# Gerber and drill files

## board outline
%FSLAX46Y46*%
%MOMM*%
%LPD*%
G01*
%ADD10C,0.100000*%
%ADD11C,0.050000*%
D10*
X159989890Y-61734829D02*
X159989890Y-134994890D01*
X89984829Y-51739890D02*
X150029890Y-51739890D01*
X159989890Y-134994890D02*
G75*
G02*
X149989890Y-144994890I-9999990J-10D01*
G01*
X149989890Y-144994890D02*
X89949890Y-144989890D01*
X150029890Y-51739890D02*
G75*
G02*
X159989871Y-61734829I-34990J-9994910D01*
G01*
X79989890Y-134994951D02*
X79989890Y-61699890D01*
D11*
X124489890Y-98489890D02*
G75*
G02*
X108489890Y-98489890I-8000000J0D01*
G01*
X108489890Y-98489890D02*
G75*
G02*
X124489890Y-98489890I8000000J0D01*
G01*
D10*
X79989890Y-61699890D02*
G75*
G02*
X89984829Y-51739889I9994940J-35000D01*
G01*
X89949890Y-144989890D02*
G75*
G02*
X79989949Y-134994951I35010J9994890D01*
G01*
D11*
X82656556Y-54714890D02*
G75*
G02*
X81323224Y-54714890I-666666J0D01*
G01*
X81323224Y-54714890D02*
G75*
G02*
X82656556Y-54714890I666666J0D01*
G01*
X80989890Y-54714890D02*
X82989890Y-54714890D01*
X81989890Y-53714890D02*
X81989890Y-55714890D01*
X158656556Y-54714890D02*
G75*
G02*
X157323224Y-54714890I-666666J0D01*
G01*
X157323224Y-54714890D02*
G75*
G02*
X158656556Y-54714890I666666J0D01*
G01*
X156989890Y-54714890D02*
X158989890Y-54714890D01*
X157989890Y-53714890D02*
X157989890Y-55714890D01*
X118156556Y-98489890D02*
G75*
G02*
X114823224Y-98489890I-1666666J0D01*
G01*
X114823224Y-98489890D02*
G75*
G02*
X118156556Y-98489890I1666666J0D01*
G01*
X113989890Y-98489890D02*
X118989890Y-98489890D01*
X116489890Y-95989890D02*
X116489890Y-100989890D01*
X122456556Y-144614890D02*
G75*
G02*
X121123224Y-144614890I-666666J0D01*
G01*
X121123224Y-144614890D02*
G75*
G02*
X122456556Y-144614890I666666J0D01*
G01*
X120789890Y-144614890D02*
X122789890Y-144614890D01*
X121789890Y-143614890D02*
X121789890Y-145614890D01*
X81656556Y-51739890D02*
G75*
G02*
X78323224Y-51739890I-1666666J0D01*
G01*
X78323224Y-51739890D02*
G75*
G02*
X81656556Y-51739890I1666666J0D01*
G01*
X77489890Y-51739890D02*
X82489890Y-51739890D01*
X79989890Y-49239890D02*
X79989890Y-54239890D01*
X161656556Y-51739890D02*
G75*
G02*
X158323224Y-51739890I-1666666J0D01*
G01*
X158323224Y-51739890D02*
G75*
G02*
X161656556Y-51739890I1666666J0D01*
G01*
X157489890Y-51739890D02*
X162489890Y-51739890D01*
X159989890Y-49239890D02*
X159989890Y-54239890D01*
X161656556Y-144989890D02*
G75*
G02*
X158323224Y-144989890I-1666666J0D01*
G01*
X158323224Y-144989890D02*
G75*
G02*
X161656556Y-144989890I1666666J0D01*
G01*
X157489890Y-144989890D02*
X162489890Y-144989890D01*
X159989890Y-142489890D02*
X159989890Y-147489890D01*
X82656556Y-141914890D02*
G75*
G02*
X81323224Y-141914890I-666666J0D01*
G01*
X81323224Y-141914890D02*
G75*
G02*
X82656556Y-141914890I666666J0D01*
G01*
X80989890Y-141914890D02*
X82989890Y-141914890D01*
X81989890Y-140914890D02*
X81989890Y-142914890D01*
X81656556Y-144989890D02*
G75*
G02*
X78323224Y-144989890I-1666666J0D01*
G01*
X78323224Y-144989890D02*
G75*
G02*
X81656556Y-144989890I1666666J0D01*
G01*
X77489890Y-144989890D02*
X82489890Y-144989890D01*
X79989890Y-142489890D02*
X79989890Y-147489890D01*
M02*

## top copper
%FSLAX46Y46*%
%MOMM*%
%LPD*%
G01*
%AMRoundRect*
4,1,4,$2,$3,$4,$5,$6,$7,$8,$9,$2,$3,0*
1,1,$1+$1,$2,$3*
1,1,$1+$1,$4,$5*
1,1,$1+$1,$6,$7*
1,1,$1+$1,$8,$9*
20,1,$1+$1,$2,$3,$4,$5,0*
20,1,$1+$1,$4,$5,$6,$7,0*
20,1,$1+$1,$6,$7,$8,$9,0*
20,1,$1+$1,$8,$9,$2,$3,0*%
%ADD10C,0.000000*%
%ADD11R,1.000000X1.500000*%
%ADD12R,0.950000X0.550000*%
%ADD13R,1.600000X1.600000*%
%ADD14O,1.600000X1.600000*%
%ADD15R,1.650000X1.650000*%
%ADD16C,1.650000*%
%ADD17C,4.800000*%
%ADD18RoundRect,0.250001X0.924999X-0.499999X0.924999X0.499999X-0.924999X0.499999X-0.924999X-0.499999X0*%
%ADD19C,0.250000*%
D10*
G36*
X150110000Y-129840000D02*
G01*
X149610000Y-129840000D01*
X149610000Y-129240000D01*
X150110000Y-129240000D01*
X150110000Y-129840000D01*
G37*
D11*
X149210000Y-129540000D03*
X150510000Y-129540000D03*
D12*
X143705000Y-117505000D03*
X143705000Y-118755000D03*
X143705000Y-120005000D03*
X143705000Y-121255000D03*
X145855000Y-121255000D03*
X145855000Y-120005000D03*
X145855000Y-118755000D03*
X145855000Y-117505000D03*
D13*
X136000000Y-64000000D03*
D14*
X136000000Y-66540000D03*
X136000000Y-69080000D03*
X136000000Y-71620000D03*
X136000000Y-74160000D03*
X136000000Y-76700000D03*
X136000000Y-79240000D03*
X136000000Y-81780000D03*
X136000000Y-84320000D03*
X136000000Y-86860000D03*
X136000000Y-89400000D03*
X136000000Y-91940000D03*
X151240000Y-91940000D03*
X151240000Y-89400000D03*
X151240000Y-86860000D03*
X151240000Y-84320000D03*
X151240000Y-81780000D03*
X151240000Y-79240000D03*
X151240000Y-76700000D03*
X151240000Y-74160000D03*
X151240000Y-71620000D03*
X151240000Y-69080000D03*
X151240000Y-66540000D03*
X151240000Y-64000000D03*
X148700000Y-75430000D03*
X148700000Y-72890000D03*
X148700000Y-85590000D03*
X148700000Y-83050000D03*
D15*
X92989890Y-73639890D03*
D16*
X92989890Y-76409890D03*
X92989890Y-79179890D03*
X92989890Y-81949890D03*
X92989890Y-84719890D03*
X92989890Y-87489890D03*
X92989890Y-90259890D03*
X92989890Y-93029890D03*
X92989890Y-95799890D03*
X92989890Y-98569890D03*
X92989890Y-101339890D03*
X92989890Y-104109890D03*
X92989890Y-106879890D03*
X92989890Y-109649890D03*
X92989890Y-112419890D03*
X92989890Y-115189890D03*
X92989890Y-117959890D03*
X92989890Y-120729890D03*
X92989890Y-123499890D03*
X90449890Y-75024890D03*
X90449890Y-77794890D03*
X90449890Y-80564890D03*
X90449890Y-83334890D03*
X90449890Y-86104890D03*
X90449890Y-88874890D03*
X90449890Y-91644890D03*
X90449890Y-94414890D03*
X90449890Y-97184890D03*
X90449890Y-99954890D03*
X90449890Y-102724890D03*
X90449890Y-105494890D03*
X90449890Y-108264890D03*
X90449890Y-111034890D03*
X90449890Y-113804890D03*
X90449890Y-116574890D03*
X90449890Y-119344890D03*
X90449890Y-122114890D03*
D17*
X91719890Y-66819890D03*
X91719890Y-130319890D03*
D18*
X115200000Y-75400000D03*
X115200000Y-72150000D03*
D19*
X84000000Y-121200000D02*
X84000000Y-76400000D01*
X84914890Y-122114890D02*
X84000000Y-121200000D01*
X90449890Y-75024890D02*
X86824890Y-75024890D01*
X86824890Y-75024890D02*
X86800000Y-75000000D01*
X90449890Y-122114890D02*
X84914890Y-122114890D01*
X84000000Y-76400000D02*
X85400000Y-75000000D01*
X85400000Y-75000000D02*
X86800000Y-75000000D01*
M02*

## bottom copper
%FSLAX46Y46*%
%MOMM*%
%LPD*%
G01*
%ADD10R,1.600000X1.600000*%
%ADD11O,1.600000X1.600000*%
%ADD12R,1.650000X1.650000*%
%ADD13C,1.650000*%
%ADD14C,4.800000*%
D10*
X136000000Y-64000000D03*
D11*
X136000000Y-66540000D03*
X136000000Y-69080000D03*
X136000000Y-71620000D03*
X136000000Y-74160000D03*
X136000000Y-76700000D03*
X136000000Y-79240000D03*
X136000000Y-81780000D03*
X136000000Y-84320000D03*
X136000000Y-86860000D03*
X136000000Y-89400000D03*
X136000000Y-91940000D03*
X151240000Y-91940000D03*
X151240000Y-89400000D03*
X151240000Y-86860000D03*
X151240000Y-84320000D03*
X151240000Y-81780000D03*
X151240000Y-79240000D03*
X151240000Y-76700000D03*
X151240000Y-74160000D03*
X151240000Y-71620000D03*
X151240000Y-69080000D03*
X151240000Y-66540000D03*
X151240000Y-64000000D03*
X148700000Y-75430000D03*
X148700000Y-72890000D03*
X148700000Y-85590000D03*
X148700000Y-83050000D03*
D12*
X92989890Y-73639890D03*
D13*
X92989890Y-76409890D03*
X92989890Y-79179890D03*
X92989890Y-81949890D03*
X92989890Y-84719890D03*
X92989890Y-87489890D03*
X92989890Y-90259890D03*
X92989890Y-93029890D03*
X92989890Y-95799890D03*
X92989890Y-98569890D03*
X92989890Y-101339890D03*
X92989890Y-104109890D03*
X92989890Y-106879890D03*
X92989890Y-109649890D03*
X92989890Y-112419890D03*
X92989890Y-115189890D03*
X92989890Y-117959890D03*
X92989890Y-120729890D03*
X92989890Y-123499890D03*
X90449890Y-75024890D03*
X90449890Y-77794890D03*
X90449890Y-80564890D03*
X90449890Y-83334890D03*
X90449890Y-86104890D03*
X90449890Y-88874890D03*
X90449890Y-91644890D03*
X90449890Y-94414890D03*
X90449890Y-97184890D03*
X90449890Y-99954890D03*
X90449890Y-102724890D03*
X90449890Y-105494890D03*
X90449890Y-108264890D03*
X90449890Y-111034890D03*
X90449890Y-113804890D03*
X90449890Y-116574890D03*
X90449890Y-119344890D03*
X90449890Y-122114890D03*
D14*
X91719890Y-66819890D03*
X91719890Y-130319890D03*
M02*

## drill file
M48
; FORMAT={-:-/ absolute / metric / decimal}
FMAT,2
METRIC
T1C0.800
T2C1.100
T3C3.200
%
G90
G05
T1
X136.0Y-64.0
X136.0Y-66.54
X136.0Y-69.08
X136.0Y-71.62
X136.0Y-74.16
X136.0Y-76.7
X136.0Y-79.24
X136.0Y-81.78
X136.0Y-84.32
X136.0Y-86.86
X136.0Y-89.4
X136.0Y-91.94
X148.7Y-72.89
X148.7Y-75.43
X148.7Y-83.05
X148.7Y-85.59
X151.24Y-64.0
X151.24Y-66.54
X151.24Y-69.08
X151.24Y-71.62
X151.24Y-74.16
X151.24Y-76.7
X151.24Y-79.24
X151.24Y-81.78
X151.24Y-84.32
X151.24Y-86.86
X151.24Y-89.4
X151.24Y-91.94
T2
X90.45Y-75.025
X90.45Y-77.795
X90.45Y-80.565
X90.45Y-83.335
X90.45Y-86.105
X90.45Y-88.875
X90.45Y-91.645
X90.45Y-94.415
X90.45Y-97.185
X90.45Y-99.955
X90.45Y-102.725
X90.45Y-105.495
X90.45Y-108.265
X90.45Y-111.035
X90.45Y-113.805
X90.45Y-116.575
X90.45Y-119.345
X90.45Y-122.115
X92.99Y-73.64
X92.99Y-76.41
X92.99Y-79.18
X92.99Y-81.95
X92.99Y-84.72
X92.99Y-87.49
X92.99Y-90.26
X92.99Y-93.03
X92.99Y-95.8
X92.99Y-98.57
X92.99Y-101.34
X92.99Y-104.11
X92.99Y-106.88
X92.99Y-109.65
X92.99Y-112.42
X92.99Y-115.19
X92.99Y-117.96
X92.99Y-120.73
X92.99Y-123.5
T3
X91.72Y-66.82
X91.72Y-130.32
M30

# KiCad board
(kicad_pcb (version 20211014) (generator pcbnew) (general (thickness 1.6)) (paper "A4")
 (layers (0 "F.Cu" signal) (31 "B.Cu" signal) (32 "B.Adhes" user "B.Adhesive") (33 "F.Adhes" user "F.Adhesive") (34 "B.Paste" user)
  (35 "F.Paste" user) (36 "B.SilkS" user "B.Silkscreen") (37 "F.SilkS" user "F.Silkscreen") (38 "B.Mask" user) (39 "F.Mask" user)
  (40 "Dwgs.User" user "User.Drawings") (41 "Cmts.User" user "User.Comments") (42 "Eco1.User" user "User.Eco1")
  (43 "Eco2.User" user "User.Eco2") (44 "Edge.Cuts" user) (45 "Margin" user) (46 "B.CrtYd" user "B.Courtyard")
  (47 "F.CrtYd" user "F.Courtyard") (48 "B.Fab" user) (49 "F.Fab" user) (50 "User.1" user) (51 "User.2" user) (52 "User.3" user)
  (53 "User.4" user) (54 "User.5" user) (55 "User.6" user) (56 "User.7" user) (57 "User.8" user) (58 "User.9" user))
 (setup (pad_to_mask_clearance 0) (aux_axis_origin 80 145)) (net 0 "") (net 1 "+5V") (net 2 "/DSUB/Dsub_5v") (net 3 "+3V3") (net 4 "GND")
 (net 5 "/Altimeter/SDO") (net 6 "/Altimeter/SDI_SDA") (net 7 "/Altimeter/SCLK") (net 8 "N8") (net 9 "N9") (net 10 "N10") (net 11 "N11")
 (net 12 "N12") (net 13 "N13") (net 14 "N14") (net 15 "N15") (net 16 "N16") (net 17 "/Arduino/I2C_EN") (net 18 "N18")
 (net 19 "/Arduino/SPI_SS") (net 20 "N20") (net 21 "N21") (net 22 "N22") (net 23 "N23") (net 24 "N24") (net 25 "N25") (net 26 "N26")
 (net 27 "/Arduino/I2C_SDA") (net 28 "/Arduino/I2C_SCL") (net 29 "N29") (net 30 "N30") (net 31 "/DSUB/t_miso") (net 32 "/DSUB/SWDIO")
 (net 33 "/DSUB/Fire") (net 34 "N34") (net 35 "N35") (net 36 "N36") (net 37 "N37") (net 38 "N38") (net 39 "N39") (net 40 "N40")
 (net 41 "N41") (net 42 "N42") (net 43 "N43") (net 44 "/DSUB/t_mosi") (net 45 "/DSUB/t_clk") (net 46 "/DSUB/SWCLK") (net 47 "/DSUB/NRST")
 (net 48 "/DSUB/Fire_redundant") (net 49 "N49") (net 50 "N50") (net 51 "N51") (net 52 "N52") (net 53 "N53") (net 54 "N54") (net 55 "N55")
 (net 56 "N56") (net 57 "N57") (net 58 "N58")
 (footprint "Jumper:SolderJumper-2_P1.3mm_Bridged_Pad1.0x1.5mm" (layer "F.Cu") (at 149.86 129.54)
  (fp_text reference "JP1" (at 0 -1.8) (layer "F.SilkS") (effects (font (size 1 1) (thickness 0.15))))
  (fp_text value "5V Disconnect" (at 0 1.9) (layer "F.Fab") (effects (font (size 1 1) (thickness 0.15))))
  (fp_poly (pts (xy -0.25 -0.3) (xy 0.25 -0.3) (xy 0.25 0.3) (xy -0.25 0.3)) (layer "F.Cu") (width 0) (fill solid))
  (pad "1" smd rect (at -0.65 0) (size 1 1.5) (layers "F.Cu" "F.Mask") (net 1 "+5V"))
  (pad "2" smd rect (at 0.65 0) (size 1 1.5) (layers "F.Cu" "F.Mask") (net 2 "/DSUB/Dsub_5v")))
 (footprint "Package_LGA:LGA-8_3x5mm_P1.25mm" (layer "F.Cu") (at 144.78 119.38)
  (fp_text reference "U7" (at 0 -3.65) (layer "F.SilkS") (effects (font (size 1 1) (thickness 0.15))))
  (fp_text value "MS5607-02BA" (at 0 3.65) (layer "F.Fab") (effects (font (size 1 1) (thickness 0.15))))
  (pad "1" smd rect (at -1.075 -1.875) (size 0.95 0.55) (layers "F.Cu" "F.Paste" "F.Mask") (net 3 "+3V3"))
  (pad "2" smd rect (at -1.075 -0.625) (size 0.95 0.55) (layers "F.Cu" "F.Paste" "F.Mask") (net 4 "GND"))
  (pad "3" smd rect (at -1.075 0.625) (size 0.95 0.55) (layers "F.Cu" "F.Paste" "F.Mask") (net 4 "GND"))
  (pad "4" smd rect (at -1.075 1.875) (size 0.95 0.55) (layers "F.Cu" "F.Paste" "F.Mask") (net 4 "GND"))
  (pad "5" smd rect (at 1.075 1.875) (size 0.95 0.55) (layers "F.Cu" "F.Paste" "F.Mask") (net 4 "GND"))
  (pad "6" smd rect (at 1.075 0.625) (size 0.95 0.55) (layers "F.Cu" "F.Paste" "F.Mask") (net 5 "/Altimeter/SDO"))
  (pad "7" smd rect (at 1.075 -0.625) (size 0.95 0.55) (layers "F.Cu" "F.Paste" "F.Mask") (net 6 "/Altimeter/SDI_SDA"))
  (pad "8" smd rect (at 1.075 -1.875) (size 0.95 0.55) (layers "F.Cu" "F.Paste" "F.Mask") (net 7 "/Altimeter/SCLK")))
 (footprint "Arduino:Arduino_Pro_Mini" (layer "F.Cu") (at 136 64)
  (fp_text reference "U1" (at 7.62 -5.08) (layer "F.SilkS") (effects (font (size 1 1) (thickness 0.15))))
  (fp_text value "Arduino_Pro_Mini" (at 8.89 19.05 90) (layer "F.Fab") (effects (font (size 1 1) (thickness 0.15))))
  (pad "1" thru_hole rect locked (at 0 0) (size 1.6 1.6) (drill 0.8) (layers *.Cu *.Mask) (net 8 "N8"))
  (pad "2" thru_hole oval locked (at 0 2.54) (size 1.6 1.6) (drill 0.8) (layers *.Cu *.Mask) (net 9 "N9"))
  (pad "3" thru_hole oval locked (at 0 5.08) (size 1.6 1.6) (drill 0.8) (layers *.Cu *.Mask) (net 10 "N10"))
  (pad "4" thru_hole oval locked (at 0 7.62) (size 1.6 1.6) (drill 0.8) (layers *.Cu *.Mask) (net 4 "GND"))
  (pad "5" thru_hole oval locked (at 0 10.16) (size 1.6 1.6) (drill 0.8) (layers *.Cu *.Mask) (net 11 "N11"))
  (pad "6" thru_hole oval locked (at 0 12.7) (size 1.6 1.6) (drill 0.8) (layers *.Cu *.Mask) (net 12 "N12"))
  (pad "7" thru_hole oval locked (at 0 15.24) (size 1.6 1.6) (drill 0.8) (layers *.Cu *.Mask) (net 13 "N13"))
  (pad "8" thru_hole oval locked (at 0 17.78) (size 1.6 1.6) (drill 0.8) (layers *.Cu *.Mask) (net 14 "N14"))
  (pad "9" thru_hole oval locked (at 0 20.32) (size 1.6 1.6) (drill 0.8) (layers *.Cu *.Mask) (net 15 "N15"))
  (pad "10" thru_hole oval locked (at 0 22.86) (size 1.6 1.6) (drill 0.8) (layers *.Cu *.Mask) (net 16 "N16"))
  (pad "11" thru_hole oval locked (at 0 25.4) (size 1.6 1.6) (drill 0.8) (layers *.Cu *.Mask) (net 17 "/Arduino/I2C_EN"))
  (pad "12" thru_hole oval locked (at 0 27.94) (size 1.6 1.6) (drill 0.8) (layers *.Cu *.Mask) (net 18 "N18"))
  (pad "13" thru_hole oval locked (at 15.24 27.94) (size 1.6 1.6) (drill 0.8) (layers *.Cu *.Mask) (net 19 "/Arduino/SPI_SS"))
  (pad "14" thru_hole oval locked (at 15.24 25.4) (size 1.6 1.6) (drill 0.8) (layers *.Cu *.Mask) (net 6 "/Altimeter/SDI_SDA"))
  (pad "15" thru_hole oval locked (at 15.24 22.86) (size 1.6 1.6) (drill 0.8) (layers *.Cu *.Mask) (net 5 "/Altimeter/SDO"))
  (pad "16" thru_hole oval locked (at 15.24 20.32) (size 1.6 1.6) (drill 0.8) (layers *.Cu *.Mask) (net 7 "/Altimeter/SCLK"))
  (pad "17" thru_hole oval locked (at 15.24 17.78) (size 1.6 1.6) (drill 0.8) (layers *.Cu *.Mask) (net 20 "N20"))
  (pad "18" thru_hole oval locked (at 15.24 15.24) (size 1.6 1.6) (drill 0.8) (layers *.Cu *.Mask) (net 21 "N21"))
  (pad "19" thru_hole oval locked (at 15.24 12.7) (size 1.6 1.6) (drill 0.8) (layers *.Cu *.Mask) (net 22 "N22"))
  (pad "20" thru_hole oval locked (at 15.24 10.16) (size 1.6 1.6) (drill 0.8) (layers *.Cu *.Mask) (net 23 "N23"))
  (pad "21" thru_hole oval locked (at 15.24 7.62) (size 1.6 1.6) (drill 0.8) (layers *.Cu *.Mask) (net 1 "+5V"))
  (pad "22" thru_hole oval locked (at 15.24 5.08) (size 1.6 1.6) (drill 0.8) (layers *.Cu *.Mask) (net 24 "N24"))
  (pad "23" thru_hole oval locked (at 15.24 2.54) (size 1.6 1.6) (drill 0.8) (layers *.Cu *.Mask) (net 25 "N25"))
  (pad "24" thru_hole oval locked (at 15.24 0) (size 1.6 1.6) (drill 0.8) (layers *.Cu *.Mask) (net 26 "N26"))
  (pad "A4" thru_hole oval locked (at 12.7 11.43) (size 1.6 1.6) (drill 0.8) (layers *.Cu *.Mask) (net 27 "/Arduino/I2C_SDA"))
  (pad "A5" thru_hole oval locked (at 12.7 8.89) (size 1.6 1.6) (drill 0.8) (layers *.Cu *.Mask) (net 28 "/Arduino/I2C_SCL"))
  (pad "A6" thru_hole oval locked (at 12.7 21.59) (size 1.6 1.6) (drill 0.8) (layers *.Cu *.Mask) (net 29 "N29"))
  (pad "A7" thru_hole oval locked (at 12.7 19.05) (size 1.6 1.6) (drill 0.8) (layers *.Cu *.Mask) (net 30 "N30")))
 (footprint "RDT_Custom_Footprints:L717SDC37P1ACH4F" (layer "F.Cu") (at 92.98989 73.63989 -90)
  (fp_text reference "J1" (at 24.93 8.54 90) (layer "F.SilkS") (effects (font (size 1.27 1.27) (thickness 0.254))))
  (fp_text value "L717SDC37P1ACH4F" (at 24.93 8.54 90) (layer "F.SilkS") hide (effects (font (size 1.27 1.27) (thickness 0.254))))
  (pad "1" thru_hole rect locked (at 0 0 270) (size 1.65 1.65) (drill 1.1) (layers *.Cu *.Mask) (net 4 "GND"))
  (pad "2" thru_hole circle locked (at 2.77 0 270) (size 1.65 1.65) (drill 1.1) (layers *.Cu *.Mask) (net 3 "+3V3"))
  (pad "3" thru_hole circle locked (at 5.54 0 270) (size 1.65 1.65) (drill 1.1) (layers *.Cu *.Mask) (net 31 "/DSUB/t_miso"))
  (pad "4" thru_hole circle locked (at 8.31 0 270) (size 1.65 1.65) (drill 1.1) (layers *.Cu *.Mask) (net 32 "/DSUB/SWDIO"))
  (pad "5" thru_hole circle locked (at 11.08 0 270) (size 1.65 1.65) (drill 1.1) (layers *.Cu *.Mask) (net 28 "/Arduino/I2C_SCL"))
  (pad "6" thru_hole circle locked (at 13.85 0 270) (size 1.65 1.65) (drill 1.1) (layers *.Cu *.Mask) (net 17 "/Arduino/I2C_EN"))
  (pad "7" thru_hole circle locked (at 16.62 0 270) (size 1.65 1.65) (drill 1.1) (layers *.Cu *.Mask) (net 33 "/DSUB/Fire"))
  (pad "8" thru_hole circle locked (at 19.39 0 270) (size 1.65 1.65) (drill 1.1) (layers *.Cu *.Mask) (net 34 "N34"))
  (pad "9" thru_hole circle locked (at 22.16 0 270) (size 1.65 1.65) (drill 1.1) (layers *.Cu *.Mask) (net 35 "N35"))
  (pad "10" thru_hole circle locked (at 24.93 0 270) (size 1.65 1.65) (drill 1.1) (layers *.Cu *.Mask) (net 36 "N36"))
  (pad "11" thru_hole circle locked (at 27.7 0 270) (size 1.65 1.65) (drill 1.1) (layers *.Cu *.Mask) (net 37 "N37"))
  (pad "12" thru_hole circle locked (at 30.47 0 270) (size 1.65 1.65) (drill 1.1) (layers *.Cu *.Mask) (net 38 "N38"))
  (pad "13" thru_hole circle locked (at 33.24 0 270) (size 1.65 1.65) (drill 1.1) (layers *.Cu *.Mask) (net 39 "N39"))
  (pad "14" thru_hole circle locked (at 36.01 0 270) (size 1.65 1.65) (drill 1.1) (layers *.Cu *.Mask) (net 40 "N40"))
  (pad "15" thru_hole circle locked (at 38.78 0 270) (size 1.65 1.65) (drill 1.1) (layers *.Cu *.Mask) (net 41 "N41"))
  (pad "16" thru_hole circle locked (at 41.55 0 270) (size 1.65 1.65) (drill 1.1) (layers *.Cu *.Mask) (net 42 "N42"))
  (pad "17" thru_hole circle locked (at 44.32 0 270) (size 1.65 1.65) (drill 1.1) (layers *.Cu *.Mask) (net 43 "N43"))
  (pad "18" thru_hole circle locked (at 47.09 0 270) (size 1.65 1.65) (drill 1.1) (layers *.Cu *.Mask) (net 3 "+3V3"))
  (pad "19" thru_hole circle locked (at 49.86 0 270) (size 1.65 1.65) (drill 1.1) (layers *.Cu *.Mask) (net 4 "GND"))
  (pad "20" thru_hole circle locked (at 1.385 2.54 270) (size 1.65 1.65) (drill 1.1) (layers *.Cu *.Mask) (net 2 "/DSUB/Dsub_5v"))
  (pad "21" thru_hole circle locked (at 4.155 2.54 270) (size 1.65 1.65) (drill 1.1) (layers *.Cu *.Mask) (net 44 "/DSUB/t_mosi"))
  (pad "22" thru_hole circle locked (at 6.925 2.54 270) (size 1.65 1.65) (drill 1.1) (layers *.Cu *.Mask) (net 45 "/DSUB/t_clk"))
  (pad "23" thru_hole circle locked (at 9.695 2.54 270) (size 1.65 1.65) (drill 1.1) (layers *.Cu *.Mask) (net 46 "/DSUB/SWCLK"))
  (pad "24" thru_hole circle locked (at 12.465 2.54 270) (size 1.65 1.65) (drill 1.1) (layers *.Cu *.Mask) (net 27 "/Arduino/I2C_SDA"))
  (pad "25" thru_hole circle locked (at 15.235 2.54 270) (size 1.65 1.65) (drill 1.1) (layers *.Cu *.Mask) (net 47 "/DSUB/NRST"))
  (pad "26" thru_hole circle locked (at 18.005 2.54 270) (size 1.65 1.65) (drill 1.1) (layers *.Cu *.Mask) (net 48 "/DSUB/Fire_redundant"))
  (pad "27" thru_hole circle locked (at 20.775 2.54 270) (size 1.65 1.65) (drill 1.1) (layers *.Cu *.Mask) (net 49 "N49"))
  (pad "28" thru_hole circle locked (at 23.545 2.54 270) (size 1.65 1.65) (drill 1.1) (layers *.Cu *.Mask) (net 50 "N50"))
  (pad "29" thru_hole circle locked (at 26.315 2.54 270) (size 1.65 1.65) (drill 1.1) (layers *.Cu *.Mask) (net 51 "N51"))
  (pad "30" thru_hole circle locked (at 29.085 2.54 270) (size 1.65 1.65) (drill 1.1) (layers *.Cu *.Mask) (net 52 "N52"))
  (pad "31" thru_hole circle locked (at 31.855 2.54 270) (size 1.65 1.65) (drill 1.1) (layers *.Cu *.Mask) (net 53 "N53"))
  (pad "32" thru_hole circle locked (at 34.625 2.54 270) (size 1.65 1.65) (drill 1.1) (layers *.Cu *.Mask) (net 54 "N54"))
  (pad "33" thru_hole circle locked (at 37.395 2.54 270) (size 1.65 1.65) (drill 1.1) (layers *.Cu *.Mask) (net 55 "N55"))
  (pad "34" thru_hole circle locked (at 40.165 2.54 270) (size 1.65 1.65) (drill 1.1) (layers *.Cu *.Mask) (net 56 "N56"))
  (pad "35" thru_hole circle locked (at 42.935 2.54 270) (size 1.65 1.65) (drill 1.1) (layers *.Cu *.Mask) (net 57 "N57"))
  (pad "36" thru_hole circle locked (at 45.705 2.54 270) (size 1.65 1.65) (drill 1.1) (layers *.Cu *.Mask) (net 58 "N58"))
  (pad "37" thru_hole circle locked (at 48.475 2.54 270) (size 1.65 1.65) (drill 1.1) (layers *.Cu *.Mask) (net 2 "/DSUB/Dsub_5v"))
  (pad "MH1" thru_hole circle locked (at -6.82 1.27 270) (size 4.8 4.8) (drill 3.2) (layers *.Cu *.Mask) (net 4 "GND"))
  (pad "MH2" thru_hole circle locked (at 56.68 1.27 270) (size 4.8 4.8) (drill 3.2) (layers *.Cu *.Mask) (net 4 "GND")))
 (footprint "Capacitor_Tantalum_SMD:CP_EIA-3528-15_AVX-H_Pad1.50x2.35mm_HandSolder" (layer "F.Cu") (at 115.2 73.775 90)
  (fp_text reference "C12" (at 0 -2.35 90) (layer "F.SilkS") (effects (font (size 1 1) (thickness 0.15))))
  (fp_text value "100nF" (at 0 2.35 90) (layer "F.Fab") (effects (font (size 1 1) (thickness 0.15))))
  (pad "1" smd roundrect (at -1.625 0 90) (size 1.5 2.35) (layers "F.Cu" "F.Paste" "F.Mask") (roundrect_rratio 0.166667) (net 3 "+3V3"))
  (pad "2" smd roundrect (at 1.625 0 90) (size 1.5 2.35) (layers "F.Cu" "F.Paste" "F.Mask") (roundrect_rratio 0.166667) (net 4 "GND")))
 (gr_line (start 159.98989 61.734829) (end 159.98989 134.99489) (layer "Edge.Cuts") (width 0.1))
 (gr_line (start 89.984829 51.73989) (end 150.02989 51.73989) (layer "Edge.Cuts") (width 0.1))
 (gr_arc (start 159.98989 134.99489) (mid 157.060958 142.065958) (end 149.98989 144.99489) (layer "Edge.Cuts") (width 0.1))
 (gr_line (start 149.98989 144.99489) (end 89.94989 144.98989) (layer "Edge.Cuts") (width 0.1))
 (gr_arc (start 150.02989 51.73989) (mid 157.074786 54.679682) (end 159.98989 61.734829) (layer "Edge.Cuts") (width 0.1))
 (gr_line (start 79.98989 134.994951) (end 79.98989 61.69989) (layer "Edge.Cuts") (width 0.1))
 (gr_circle (center 116.48989 98.48989) (end 124.48989 98.48989) (layer "Edge.Cuts") (width 0.05) (fill none))
 (gr_arc (start 79.98989 61.69989) (mid 82.929682 54.654994) (end 89.984829 51.73989) (layer "Edge.Cuts") (width 0.1))
 (gr_arc (start 89.94989 144.98989) (mid 82.904994 142.050098) (end 79.98989 134.994951) (layer "Edge.Cuts") (width 0.1))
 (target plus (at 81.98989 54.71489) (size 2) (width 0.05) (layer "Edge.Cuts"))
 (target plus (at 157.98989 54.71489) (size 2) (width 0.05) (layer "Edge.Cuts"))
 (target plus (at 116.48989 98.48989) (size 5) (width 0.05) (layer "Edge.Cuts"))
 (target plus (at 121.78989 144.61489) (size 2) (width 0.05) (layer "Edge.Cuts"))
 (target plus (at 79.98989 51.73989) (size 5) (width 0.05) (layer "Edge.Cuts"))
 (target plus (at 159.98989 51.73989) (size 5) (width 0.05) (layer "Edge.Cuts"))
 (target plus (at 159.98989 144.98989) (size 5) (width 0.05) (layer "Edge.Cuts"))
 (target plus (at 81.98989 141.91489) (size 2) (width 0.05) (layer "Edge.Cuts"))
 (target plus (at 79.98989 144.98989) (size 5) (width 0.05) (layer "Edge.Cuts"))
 (segment (start 84 121.2) (end 84 76.4) (width 0.25) (layer "F.Cu") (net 2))
 (segment (start 84.91489 122.11489) (end 84 121.2) (width 0.25) (layer "F.Cu") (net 2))
 (segment (start 90.44989 75.02489) (end 86.82489 75.02489) (width 0.25) (layer "F.Cu") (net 2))
 (segment (start 86.82489 75.02489) (end 86.8 75) (width 0.25) (layer "F.Cu") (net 2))
 (segment (start 90.44989 122.11489) (end 84.91489 122.11489) (width 0.25) (layer "F.Cu") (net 2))
 (segment (start 84 76.4) (end 85.4 75) (width 0.25) (layer "F.Cu") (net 2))
 (segment (start 85.4 75) (end 86.8 75) (width 0.25) (layer "F.Cu") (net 2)))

